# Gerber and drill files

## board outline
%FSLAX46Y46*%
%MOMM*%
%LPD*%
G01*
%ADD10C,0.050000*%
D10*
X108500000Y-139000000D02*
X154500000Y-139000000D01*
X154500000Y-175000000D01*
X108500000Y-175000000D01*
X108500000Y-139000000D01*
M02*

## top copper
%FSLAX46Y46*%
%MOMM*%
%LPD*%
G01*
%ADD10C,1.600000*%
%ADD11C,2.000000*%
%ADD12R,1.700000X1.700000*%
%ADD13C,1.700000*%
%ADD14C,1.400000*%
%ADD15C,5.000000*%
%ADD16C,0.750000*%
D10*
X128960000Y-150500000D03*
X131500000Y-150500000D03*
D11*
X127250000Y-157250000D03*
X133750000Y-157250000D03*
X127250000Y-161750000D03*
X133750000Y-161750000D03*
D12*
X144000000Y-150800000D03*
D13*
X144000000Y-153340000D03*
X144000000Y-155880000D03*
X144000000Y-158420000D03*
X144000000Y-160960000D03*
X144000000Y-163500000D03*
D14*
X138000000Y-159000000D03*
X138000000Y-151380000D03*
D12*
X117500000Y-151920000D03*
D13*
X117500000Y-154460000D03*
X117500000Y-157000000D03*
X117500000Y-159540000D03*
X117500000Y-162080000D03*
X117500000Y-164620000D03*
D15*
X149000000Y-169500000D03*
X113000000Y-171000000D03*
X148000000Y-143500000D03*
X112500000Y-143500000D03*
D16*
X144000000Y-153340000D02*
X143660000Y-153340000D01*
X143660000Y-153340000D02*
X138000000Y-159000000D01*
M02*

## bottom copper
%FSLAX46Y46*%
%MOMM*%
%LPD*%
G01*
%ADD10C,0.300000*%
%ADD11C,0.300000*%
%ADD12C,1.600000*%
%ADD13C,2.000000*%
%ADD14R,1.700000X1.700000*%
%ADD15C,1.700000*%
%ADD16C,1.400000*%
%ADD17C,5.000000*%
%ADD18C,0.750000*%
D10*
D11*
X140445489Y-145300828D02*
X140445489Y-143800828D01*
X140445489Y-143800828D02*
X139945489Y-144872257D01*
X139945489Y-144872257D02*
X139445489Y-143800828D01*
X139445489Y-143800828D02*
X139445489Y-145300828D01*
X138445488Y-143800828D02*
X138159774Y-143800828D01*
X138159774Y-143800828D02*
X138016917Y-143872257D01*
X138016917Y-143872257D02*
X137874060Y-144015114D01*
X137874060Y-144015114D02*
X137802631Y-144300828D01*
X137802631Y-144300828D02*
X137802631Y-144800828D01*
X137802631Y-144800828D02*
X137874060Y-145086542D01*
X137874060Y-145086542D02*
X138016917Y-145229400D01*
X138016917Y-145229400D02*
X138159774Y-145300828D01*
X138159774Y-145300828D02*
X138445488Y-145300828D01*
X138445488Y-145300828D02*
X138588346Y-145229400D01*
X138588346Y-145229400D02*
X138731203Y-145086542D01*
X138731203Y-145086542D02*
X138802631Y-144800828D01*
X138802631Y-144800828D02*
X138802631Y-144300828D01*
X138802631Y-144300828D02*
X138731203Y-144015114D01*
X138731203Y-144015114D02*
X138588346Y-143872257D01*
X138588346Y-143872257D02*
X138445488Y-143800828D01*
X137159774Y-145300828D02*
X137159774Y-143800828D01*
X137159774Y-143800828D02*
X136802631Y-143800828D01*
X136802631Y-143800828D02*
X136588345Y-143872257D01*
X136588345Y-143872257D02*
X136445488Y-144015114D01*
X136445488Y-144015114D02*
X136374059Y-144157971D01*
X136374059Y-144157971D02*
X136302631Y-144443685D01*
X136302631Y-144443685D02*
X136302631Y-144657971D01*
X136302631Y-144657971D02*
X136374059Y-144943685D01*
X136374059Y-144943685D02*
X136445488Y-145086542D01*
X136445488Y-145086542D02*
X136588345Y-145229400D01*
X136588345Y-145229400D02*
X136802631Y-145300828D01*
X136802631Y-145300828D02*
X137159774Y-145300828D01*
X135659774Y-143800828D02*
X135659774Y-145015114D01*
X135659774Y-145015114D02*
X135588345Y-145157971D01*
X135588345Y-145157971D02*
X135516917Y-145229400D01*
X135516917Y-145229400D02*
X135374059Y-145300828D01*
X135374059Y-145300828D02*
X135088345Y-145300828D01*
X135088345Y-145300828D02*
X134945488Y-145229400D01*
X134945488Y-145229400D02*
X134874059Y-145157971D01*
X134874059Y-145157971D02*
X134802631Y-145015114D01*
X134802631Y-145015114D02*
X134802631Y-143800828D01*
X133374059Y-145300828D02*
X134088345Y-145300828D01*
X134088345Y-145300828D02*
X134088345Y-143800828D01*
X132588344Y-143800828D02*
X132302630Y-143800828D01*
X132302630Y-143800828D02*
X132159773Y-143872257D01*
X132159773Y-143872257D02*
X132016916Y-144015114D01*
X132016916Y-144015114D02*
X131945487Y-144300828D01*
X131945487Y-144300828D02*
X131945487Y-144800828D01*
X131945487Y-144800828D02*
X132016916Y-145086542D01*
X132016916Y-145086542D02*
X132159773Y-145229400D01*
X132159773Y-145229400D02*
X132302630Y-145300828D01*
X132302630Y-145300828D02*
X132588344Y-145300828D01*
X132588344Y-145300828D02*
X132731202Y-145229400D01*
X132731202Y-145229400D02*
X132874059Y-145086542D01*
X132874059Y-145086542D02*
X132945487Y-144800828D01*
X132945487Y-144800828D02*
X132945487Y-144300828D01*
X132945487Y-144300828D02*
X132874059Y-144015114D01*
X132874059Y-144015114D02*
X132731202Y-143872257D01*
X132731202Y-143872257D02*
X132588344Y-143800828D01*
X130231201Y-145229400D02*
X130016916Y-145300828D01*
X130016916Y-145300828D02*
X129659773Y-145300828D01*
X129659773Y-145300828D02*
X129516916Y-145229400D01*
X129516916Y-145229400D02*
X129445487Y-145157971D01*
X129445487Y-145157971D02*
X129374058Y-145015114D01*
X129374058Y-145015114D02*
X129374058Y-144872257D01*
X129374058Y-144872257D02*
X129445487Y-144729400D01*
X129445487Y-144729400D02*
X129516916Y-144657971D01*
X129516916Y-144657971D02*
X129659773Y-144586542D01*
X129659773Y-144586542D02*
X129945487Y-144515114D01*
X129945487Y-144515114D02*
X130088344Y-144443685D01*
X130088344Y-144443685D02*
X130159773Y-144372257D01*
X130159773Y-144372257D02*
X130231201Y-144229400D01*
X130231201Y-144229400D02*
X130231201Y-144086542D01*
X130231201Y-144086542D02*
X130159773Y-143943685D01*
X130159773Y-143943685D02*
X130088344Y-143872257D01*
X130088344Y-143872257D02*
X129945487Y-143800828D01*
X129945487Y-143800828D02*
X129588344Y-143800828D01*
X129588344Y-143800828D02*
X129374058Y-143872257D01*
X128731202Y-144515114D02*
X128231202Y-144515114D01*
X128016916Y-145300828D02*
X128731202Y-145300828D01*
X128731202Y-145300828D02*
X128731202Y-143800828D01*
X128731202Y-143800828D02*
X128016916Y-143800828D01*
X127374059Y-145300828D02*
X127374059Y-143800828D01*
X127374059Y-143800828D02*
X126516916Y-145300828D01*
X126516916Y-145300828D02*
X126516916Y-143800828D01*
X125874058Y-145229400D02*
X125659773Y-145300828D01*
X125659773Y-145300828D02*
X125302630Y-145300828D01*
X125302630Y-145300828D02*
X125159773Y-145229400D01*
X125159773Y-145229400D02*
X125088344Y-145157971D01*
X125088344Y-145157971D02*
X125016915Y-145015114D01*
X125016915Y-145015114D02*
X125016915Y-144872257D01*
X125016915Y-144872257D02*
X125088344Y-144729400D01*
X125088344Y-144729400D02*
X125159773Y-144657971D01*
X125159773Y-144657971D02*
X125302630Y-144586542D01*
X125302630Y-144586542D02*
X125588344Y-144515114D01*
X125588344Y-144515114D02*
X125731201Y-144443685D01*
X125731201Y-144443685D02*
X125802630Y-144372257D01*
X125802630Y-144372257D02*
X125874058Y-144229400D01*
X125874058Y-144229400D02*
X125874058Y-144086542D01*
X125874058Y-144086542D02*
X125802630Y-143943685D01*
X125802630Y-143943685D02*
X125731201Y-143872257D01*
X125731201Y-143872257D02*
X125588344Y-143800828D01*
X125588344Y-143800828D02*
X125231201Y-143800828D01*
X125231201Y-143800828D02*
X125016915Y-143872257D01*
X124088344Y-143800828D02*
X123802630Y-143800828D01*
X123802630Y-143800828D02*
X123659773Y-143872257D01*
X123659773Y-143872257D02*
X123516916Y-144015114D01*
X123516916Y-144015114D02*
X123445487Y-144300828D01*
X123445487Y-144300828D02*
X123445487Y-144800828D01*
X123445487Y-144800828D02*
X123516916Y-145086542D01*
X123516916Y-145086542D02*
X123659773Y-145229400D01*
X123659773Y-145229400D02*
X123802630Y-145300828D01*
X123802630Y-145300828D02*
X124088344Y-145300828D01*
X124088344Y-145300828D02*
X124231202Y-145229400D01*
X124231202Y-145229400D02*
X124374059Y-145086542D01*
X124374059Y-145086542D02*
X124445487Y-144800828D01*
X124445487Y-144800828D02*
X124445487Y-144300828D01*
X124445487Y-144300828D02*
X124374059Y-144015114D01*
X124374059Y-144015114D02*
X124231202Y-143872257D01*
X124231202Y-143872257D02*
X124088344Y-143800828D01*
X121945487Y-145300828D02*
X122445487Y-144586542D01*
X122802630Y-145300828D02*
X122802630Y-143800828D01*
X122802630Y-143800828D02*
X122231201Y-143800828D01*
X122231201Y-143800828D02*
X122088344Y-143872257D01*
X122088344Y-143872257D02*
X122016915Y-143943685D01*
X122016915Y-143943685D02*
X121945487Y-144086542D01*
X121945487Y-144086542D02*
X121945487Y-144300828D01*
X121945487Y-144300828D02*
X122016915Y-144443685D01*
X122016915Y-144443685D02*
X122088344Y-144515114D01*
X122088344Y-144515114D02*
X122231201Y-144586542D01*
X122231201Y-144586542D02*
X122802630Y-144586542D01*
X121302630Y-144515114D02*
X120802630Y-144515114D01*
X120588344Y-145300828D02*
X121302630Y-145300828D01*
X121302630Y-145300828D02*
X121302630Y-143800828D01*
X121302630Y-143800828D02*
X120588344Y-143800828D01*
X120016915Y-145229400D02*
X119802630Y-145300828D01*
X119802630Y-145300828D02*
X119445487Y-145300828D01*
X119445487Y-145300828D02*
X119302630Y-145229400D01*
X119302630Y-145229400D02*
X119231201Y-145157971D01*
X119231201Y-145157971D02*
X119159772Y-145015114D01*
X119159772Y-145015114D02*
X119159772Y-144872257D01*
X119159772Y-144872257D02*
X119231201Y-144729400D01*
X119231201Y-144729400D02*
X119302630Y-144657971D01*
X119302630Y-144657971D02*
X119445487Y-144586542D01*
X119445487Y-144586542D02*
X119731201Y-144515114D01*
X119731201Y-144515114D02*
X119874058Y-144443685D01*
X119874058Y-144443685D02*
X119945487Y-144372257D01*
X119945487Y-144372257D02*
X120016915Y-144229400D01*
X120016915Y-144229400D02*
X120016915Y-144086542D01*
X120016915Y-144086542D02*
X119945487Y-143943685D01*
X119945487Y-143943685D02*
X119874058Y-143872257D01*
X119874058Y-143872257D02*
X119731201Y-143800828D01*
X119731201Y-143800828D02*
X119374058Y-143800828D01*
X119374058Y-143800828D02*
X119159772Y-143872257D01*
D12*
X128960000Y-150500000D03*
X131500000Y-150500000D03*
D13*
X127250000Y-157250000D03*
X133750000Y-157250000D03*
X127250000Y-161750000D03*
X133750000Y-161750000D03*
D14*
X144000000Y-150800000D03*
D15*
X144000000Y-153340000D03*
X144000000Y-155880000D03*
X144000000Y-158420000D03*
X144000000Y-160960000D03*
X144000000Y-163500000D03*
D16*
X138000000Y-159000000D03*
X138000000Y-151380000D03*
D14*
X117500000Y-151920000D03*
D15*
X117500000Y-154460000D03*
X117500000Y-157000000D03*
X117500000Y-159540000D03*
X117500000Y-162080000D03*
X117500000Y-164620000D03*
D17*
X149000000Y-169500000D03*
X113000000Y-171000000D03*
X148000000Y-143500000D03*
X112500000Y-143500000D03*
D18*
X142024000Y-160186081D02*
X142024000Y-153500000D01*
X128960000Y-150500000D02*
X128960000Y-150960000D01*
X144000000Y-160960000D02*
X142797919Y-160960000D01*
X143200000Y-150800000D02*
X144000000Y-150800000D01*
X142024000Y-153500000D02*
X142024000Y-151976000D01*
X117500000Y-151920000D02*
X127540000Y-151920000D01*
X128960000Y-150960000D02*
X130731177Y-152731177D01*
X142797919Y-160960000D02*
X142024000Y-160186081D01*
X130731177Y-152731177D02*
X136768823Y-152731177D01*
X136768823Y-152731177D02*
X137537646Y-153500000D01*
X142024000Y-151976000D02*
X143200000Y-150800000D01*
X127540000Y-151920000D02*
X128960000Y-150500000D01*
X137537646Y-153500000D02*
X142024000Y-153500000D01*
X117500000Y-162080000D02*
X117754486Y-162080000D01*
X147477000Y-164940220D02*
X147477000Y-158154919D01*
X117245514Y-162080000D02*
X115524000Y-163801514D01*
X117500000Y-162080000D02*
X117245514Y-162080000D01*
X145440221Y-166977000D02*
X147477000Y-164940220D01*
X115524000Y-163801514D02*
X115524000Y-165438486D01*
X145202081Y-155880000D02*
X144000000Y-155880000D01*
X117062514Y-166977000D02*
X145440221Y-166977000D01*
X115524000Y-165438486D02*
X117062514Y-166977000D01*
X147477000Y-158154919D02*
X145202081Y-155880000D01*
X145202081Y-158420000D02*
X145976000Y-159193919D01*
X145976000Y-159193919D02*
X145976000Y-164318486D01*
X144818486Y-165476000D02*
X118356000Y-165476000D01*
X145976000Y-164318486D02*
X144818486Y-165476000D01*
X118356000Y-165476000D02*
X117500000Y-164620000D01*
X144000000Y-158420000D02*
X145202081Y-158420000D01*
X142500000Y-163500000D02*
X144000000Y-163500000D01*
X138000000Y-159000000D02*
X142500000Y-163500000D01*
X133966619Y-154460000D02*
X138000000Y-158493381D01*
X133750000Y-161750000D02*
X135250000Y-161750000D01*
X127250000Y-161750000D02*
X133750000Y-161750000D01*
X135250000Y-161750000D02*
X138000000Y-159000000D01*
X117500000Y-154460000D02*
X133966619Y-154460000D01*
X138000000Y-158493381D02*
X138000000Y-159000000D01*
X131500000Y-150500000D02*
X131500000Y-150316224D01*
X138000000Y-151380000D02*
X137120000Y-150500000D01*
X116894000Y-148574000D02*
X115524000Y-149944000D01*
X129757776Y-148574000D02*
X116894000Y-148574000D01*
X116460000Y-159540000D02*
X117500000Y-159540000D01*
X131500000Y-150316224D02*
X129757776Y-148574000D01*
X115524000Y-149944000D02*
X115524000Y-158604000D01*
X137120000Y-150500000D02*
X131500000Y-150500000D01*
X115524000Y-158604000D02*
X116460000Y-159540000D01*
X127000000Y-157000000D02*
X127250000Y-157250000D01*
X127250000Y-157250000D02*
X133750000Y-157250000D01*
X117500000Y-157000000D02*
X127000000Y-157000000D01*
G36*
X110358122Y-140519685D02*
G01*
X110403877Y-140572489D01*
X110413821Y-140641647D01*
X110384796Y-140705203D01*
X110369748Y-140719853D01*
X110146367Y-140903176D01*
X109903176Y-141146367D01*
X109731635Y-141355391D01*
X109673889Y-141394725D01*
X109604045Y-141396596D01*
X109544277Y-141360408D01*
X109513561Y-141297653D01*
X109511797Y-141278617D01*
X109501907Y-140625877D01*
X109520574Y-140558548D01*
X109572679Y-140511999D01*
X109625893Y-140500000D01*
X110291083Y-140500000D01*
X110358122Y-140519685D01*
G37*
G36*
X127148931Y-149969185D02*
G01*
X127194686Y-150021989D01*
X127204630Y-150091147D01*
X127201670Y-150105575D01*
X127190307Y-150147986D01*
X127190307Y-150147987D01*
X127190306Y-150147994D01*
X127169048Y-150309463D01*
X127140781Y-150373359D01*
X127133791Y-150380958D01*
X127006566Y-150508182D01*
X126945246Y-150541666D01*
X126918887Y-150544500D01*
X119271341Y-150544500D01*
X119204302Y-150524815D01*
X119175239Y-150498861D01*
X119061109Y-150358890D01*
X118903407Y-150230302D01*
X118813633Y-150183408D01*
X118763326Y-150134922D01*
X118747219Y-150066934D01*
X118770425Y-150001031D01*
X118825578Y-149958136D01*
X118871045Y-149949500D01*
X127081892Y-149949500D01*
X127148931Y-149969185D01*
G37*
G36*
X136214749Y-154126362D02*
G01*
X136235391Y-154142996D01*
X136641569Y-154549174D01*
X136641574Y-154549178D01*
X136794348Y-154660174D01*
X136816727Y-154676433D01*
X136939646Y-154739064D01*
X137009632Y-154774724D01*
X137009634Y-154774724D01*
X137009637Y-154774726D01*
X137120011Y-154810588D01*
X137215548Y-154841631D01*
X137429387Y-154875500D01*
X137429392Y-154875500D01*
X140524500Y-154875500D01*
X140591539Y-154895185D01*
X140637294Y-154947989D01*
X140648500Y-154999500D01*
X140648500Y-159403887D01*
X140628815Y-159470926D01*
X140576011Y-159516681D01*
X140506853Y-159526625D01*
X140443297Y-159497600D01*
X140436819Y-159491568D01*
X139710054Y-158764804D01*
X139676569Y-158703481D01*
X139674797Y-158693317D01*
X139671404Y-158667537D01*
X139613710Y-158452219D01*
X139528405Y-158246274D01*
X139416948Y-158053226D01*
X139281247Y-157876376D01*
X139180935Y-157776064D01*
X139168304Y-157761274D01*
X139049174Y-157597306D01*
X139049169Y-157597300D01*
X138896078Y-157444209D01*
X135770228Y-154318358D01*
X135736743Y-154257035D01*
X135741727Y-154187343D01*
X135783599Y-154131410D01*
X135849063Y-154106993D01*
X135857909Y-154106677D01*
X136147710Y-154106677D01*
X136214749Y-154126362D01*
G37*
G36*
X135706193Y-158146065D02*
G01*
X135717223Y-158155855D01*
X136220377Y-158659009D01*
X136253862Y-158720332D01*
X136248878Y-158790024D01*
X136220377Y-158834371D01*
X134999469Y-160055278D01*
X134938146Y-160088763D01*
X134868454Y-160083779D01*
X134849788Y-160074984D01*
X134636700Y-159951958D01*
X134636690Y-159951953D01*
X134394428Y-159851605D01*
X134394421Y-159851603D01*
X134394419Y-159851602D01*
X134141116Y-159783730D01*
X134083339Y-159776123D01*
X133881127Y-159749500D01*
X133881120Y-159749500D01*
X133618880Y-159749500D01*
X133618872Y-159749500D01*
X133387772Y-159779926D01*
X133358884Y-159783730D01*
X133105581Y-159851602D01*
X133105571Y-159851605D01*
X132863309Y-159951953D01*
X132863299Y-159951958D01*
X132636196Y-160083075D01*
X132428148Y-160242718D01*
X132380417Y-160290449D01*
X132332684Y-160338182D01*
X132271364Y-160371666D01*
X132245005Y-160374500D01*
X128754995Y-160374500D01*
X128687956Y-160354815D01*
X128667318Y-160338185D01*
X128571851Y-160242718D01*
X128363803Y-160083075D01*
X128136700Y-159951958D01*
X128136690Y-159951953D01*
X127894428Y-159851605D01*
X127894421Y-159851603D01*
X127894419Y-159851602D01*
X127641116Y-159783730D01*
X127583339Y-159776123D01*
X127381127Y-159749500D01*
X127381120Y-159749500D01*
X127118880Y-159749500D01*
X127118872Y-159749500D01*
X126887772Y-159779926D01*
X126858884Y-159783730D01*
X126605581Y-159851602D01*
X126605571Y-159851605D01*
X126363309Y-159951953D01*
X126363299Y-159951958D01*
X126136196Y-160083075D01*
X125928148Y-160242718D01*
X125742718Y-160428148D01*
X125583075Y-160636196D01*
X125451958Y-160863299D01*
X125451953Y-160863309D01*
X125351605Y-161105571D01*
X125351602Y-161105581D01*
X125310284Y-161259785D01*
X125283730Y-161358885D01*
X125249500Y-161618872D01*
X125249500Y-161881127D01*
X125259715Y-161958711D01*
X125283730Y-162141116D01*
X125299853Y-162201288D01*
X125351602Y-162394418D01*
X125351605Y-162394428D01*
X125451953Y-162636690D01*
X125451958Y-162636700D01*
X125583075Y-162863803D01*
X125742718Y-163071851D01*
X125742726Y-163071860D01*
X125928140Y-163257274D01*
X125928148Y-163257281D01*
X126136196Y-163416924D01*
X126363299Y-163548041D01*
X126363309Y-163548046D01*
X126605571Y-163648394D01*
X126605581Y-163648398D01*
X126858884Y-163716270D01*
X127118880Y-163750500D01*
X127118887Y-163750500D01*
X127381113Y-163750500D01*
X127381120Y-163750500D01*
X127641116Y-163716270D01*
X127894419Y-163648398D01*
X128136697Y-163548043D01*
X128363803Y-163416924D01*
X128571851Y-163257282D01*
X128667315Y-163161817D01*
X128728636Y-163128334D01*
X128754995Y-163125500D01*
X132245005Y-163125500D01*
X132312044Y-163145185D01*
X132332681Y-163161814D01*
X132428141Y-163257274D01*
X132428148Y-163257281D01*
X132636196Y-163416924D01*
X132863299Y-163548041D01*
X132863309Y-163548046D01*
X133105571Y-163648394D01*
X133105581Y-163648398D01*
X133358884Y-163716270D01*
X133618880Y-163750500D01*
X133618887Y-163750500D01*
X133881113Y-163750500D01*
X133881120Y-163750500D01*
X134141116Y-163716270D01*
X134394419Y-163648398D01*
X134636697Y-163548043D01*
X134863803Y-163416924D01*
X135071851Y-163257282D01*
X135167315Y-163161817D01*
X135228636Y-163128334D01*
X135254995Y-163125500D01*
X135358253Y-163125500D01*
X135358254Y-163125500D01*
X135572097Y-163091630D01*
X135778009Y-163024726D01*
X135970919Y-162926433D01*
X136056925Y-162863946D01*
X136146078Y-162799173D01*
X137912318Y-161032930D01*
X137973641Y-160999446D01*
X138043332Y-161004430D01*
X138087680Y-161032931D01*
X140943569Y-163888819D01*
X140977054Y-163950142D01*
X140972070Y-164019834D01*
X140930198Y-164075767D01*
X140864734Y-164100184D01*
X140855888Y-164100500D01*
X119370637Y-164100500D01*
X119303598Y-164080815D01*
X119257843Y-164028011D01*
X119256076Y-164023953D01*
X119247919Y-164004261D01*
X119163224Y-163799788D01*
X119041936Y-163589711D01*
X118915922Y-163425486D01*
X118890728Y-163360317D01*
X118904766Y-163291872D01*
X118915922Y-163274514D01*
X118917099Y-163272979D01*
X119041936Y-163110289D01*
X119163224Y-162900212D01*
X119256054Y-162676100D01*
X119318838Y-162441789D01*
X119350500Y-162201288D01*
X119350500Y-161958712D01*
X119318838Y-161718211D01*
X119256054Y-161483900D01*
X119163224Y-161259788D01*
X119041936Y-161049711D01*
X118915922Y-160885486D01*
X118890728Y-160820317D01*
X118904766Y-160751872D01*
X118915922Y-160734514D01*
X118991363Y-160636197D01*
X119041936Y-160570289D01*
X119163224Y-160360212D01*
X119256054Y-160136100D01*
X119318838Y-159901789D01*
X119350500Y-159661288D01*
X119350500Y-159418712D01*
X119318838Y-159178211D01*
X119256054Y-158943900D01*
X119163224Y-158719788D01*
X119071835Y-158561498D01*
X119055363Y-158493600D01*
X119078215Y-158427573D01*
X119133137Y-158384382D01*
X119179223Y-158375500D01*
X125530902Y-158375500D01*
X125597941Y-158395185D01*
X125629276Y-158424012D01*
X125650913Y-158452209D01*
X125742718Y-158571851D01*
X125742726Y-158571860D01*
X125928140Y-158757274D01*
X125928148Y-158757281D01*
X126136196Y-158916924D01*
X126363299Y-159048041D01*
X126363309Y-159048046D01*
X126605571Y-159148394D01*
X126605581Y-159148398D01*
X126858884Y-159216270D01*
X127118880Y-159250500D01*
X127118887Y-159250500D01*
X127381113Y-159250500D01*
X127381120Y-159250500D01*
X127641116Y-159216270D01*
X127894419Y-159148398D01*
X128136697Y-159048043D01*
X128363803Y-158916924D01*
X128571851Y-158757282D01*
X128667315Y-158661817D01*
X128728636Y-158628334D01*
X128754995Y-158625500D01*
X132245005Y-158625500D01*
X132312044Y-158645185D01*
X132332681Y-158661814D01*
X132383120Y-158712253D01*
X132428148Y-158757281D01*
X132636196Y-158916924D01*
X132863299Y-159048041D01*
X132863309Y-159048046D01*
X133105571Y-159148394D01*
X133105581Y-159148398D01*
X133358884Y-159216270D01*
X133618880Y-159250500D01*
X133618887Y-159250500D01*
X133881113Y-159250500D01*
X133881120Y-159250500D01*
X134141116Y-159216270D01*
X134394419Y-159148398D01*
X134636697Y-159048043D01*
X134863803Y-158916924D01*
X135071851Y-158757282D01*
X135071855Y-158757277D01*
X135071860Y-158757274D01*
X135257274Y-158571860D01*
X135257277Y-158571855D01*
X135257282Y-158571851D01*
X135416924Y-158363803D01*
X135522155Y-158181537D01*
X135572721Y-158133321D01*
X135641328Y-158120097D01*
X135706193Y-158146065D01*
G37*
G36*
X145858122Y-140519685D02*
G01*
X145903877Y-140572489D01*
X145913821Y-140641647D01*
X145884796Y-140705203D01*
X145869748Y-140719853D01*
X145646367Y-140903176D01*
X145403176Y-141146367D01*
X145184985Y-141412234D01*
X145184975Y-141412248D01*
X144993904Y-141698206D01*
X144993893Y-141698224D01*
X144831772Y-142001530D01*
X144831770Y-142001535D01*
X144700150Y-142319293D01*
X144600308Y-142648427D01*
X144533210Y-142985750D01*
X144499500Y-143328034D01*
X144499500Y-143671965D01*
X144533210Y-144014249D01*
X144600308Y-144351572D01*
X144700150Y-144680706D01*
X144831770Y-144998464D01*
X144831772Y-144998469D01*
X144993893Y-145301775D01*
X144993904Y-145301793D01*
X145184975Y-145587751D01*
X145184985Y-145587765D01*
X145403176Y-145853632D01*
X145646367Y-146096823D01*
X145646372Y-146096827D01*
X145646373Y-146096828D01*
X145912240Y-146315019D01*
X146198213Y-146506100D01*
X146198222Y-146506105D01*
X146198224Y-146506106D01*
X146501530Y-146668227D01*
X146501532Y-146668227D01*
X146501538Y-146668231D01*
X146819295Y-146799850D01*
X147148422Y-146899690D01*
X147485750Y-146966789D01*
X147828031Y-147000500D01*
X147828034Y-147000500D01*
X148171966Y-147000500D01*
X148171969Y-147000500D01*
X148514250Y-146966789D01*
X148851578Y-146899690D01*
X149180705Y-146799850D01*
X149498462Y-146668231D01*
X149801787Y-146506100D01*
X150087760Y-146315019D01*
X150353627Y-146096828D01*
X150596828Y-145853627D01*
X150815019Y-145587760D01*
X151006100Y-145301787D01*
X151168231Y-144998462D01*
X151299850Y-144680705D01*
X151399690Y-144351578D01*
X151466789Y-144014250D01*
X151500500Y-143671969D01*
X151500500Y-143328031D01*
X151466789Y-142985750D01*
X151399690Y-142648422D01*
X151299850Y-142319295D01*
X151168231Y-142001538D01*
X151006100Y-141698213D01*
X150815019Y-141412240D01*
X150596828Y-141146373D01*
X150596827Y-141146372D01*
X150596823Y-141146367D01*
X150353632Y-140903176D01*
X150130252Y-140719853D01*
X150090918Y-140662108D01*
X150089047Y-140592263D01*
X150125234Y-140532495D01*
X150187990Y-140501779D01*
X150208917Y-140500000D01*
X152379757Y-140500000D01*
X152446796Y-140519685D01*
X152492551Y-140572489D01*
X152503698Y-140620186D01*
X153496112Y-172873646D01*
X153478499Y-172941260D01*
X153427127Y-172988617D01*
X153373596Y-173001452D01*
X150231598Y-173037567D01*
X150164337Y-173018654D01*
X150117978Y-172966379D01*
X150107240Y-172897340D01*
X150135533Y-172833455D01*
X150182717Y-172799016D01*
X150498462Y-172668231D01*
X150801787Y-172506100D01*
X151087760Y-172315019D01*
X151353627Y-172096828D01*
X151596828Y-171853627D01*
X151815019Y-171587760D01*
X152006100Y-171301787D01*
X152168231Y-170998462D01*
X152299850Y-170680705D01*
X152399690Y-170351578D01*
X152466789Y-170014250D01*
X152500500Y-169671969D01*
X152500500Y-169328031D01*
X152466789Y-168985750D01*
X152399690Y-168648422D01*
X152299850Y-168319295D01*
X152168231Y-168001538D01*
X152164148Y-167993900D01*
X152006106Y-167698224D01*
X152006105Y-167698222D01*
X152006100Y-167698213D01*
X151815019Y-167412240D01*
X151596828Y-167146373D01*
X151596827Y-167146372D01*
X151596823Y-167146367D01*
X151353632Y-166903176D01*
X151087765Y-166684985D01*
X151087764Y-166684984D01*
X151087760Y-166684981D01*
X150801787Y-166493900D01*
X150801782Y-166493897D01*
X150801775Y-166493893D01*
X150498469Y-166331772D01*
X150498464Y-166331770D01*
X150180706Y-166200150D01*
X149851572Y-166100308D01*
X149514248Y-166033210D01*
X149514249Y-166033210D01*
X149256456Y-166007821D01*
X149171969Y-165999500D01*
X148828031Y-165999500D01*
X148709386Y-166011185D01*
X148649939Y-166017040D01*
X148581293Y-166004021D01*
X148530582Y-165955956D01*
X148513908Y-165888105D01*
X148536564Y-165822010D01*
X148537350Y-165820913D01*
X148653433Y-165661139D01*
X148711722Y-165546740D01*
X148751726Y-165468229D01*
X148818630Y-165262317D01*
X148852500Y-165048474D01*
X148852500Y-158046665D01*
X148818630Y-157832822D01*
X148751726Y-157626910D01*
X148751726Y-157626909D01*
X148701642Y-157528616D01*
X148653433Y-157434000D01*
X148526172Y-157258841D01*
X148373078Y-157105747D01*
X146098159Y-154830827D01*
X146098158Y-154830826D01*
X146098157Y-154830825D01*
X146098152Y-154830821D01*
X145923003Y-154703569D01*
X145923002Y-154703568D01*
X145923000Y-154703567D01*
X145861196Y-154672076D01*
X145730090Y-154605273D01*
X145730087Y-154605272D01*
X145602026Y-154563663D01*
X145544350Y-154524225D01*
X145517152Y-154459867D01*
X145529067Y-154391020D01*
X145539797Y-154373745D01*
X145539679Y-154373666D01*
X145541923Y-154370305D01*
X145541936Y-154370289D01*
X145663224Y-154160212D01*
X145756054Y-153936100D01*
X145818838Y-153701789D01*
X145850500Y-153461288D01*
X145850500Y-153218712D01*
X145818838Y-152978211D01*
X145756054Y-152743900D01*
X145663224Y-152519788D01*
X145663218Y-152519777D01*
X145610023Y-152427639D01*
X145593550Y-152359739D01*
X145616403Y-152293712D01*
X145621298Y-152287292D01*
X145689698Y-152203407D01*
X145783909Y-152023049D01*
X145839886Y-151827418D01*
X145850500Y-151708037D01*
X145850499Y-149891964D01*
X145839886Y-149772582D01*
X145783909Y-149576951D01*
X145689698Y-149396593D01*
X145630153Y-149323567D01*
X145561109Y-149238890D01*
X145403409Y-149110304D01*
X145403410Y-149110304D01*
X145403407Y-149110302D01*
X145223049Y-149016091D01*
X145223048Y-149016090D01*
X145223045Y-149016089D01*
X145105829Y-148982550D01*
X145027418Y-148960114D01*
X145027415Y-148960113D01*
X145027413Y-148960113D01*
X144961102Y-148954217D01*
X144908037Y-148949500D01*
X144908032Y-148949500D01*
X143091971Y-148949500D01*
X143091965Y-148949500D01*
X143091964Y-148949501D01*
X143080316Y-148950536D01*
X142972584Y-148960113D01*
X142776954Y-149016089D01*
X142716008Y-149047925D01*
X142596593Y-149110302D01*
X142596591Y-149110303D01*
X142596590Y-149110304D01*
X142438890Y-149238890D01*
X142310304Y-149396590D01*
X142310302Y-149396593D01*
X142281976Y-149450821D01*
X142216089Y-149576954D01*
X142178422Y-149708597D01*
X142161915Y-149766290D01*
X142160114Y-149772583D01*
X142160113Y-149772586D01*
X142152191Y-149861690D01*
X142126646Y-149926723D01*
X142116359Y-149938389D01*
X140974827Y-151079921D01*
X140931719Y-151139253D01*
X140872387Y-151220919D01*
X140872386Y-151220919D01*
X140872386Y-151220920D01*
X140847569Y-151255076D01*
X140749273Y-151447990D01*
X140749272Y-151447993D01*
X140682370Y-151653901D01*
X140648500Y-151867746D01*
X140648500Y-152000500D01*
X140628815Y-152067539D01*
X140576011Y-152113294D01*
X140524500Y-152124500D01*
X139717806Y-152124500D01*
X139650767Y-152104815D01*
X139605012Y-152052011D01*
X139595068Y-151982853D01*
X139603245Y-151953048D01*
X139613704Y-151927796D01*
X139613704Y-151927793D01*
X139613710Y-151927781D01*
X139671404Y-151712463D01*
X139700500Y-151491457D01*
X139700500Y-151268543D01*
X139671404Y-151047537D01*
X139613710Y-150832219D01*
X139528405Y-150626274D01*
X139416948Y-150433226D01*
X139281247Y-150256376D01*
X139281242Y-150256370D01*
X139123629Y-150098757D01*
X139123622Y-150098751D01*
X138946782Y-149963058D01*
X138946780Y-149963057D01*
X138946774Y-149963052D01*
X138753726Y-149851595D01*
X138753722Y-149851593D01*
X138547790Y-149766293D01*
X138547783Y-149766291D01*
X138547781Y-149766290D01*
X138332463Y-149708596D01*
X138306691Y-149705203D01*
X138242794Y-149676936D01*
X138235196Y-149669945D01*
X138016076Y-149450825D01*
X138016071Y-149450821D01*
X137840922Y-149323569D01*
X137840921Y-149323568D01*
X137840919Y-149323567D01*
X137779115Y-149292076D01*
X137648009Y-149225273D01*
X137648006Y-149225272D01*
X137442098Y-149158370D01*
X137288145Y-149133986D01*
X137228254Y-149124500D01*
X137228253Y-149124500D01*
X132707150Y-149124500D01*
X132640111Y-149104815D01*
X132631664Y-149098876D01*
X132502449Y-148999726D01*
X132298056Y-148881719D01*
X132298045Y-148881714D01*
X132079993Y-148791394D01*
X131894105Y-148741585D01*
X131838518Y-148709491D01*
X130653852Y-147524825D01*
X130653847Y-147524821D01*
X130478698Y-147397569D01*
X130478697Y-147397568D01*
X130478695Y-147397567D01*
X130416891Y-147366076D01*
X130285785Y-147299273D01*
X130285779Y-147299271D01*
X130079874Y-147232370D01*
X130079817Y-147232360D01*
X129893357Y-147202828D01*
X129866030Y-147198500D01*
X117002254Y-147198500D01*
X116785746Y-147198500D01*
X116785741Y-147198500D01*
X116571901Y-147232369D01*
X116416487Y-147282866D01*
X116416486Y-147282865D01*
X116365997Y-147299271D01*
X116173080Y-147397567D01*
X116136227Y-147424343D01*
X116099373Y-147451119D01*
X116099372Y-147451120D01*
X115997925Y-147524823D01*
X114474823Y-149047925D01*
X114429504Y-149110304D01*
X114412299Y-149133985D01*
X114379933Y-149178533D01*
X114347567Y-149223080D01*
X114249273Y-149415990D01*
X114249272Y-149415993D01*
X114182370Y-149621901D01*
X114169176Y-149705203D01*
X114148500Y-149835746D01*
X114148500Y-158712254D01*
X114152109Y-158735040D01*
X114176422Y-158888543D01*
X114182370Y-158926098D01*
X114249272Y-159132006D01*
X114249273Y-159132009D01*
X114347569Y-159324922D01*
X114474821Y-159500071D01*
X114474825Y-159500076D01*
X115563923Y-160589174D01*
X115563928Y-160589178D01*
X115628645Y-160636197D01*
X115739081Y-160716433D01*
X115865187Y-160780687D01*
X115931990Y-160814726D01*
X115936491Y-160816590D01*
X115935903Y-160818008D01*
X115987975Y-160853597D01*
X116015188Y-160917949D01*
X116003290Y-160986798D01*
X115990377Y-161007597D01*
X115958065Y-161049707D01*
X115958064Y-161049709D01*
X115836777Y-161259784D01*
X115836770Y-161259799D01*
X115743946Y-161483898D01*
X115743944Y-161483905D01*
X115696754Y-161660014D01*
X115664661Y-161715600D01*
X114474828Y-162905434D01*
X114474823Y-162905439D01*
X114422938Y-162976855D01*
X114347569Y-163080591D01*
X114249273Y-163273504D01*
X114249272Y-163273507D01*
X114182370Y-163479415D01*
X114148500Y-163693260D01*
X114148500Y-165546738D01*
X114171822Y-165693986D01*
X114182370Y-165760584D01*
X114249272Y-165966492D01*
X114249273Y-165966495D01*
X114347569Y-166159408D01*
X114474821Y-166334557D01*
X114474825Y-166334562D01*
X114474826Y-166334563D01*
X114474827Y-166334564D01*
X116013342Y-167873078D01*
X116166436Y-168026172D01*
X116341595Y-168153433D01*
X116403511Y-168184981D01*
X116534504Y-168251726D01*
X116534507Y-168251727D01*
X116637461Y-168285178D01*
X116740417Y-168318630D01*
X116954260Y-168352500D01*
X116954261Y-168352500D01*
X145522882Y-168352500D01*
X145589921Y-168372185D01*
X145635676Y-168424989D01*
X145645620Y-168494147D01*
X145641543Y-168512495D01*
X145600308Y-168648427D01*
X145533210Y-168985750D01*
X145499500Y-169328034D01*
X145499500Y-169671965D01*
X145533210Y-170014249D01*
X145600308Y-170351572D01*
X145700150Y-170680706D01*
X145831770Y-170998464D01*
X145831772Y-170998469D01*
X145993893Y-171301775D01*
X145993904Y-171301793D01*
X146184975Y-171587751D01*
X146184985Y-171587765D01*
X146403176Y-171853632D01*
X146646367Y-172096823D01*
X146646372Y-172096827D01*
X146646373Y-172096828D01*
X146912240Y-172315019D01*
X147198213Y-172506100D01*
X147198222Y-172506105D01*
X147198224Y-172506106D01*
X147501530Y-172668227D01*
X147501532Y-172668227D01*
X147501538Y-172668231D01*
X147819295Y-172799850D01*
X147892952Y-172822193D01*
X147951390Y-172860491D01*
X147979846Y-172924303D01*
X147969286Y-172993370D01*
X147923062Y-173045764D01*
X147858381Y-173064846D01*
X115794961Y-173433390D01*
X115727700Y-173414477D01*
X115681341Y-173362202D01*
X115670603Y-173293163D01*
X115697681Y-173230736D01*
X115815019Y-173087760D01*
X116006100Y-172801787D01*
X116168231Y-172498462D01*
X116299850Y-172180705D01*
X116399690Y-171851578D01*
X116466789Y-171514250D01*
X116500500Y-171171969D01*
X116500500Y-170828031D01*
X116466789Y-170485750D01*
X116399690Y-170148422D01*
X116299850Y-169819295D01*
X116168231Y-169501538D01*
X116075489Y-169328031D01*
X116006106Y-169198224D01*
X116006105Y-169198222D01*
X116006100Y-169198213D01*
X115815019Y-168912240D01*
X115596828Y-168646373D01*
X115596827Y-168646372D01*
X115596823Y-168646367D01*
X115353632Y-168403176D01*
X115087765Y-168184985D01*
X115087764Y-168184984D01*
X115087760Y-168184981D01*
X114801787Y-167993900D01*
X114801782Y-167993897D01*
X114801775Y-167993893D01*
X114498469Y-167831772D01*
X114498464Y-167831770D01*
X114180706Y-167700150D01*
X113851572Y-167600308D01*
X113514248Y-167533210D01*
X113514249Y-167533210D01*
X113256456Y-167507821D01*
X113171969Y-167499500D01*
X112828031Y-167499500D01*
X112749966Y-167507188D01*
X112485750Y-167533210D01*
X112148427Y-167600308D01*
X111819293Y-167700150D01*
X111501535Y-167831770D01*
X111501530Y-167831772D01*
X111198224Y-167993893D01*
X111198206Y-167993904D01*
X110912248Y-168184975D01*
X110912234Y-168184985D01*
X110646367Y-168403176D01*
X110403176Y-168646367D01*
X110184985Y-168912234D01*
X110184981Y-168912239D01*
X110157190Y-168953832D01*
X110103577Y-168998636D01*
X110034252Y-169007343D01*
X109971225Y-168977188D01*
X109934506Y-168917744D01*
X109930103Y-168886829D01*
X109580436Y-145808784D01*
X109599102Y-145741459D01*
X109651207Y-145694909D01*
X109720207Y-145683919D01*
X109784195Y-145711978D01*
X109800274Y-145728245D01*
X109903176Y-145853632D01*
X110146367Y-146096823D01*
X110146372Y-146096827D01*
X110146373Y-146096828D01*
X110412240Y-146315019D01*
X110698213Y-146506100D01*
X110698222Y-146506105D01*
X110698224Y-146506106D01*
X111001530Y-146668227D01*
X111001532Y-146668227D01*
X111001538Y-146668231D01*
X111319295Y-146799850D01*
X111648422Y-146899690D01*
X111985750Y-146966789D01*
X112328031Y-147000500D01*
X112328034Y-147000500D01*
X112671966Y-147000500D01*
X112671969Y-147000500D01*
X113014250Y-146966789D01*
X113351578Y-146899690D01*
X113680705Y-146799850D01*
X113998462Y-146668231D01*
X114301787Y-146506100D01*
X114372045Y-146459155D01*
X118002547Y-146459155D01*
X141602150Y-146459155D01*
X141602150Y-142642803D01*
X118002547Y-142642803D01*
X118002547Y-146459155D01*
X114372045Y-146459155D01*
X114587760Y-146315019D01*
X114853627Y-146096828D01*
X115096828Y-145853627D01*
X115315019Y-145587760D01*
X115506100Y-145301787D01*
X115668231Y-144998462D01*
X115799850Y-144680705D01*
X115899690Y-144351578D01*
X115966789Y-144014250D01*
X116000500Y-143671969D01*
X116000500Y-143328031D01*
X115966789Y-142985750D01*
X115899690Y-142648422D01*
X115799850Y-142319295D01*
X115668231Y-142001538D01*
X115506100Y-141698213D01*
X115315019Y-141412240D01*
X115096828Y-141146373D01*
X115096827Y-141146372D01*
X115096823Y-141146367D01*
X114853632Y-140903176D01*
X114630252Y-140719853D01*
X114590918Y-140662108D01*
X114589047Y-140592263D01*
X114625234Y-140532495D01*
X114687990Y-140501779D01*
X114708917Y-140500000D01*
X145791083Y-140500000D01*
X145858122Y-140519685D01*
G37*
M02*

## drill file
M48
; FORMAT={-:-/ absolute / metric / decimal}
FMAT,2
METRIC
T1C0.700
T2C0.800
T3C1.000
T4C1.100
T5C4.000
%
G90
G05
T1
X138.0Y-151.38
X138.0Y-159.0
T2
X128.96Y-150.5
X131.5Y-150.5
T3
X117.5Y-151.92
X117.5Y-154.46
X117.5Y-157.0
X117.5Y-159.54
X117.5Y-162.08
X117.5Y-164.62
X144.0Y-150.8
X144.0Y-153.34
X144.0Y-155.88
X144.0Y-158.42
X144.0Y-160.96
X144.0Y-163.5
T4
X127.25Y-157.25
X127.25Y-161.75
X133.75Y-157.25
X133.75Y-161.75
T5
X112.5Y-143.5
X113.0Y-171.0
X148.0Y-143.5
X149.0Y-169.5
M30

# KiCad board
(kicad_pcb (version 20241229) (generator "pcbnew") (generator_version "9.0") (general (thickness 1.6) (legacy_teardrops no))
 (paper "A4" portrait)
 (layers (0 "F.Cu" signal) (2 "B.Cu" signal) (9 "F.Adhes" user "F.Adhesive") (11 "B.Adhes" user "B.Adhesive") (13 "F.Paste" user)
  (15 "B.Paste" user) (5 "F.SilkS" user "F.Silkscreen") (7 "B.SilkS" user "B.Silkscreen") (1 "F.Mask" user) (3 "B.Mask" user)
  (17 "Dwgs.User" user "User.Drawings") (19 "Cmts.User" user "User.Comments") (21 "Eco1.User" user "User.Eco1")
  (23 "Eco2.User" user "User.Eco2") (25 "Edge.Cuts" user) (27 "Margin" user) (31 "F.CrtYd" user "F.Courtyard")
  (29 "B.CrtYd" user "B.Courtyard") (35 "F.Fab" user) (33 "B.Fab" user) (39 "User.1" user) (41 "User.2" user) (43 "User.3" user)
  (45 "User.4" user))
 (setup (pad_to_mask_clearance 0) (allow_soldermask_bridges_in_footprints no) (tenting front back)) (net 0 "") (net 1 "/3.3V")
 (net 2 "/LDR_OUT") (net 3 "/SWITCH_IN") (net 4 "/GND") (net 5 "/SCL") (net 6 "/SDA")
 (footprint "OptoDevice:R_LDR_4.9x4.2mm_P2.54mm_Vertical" (layer "F.Cu") (at 128.96 150.5)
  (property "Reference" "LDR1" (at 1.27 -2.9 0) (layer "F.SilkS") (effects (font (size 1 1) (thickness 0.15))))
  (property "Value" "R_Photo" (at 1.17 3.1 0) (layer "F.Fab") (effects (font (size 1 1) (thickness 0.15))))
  (pad "1" thru_hole circle (at 0 0) (size 1.6 1.6) (drill 0.8) (layers "*.Cu" "*.Mask") (remove_unused_layers no) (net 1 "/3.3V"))
  (pad "2" thru_hole circle (at 2.54 0) (size 1.6 1.6) (drill 0.8) (layers "*.Cu" "*.Mask") (remove_unused_layers no) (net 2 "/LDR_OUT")))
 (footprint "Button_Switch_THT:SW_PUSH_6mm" (layer "F.Cu") (at 127.25 157.25)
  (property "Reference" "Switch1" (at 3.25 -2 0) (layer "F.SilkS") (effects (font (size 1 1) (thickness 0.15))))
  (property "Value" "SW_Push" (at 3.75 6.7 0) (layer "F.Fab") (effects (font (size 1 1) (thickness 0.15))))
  (pad "1" thru_hole circle (at 0 0 90) (size 2 2) (drill 1.1) (layers "*.Cu" "*.Mask") (remove_unused_layers no) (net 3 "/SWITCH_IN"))
  (pad "1" thru_hole circle (at 6.5 0 90) (size 2 2) (drill 1.1) (layers "*.Cu" "*.Mask") (remove_unused_layers no) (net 3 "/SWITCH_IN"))
  (pad "2" thru_hole circle (at 0 4.5 90) (size 2 2) (drill 1.1) (layers "*.Cu" "*.Mask") (remove_unused_layers no) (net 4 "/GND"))
  (pad "2" thru_hole circle (at 6.5 4.5 90) (size 2 2) (drill 1.1) (layers "*.Cu" "*.Mask") (remove_unused_layers no) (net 4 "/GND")))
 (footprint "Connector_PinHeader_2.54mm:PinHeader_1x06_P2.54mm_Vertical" (layer "F.Cu") (at 144 150.8)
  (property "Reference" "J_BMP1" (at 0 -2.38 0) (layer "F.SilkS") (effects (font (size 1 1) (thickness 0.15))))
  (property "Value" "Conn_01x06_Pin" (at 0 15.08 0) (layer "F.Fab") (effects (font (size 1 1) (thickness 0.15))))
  (pad "1" thru_hole rect (at 0 0) (size 1.7 1.7) (drill 1) (layers "*.Cu" "*.Mask") (remove_unused_layers no) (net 1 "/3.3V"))
  (pad "2" thru_hole circle (at 0 2.54) (size 1.7 1.7) (drill 1) (layers "*.Cu" "*.Mask") (remove_unused_layers no) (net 4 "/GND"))
  (pad "3" thru_hole circle (at 0 5.08) (size 1.7 1.7) (drill 1) (layers "*.Cu" "*.Mask") (remove_unused_layers no) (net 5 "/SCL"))
  (pad "4" thru_hole circle (at 0 7.62) (size 1.7 1.7) (drill 1) (layers "*.Cu" "*.Mask") (remove_unused_layers no) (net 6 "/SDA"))
  (pad "5" thru_hole circle (at 0 10.16) (size 1.7 1.7) (drill 1) (layers "*.Cu" "*.Mask") (remove_unused_layers no) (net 1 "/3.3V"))
  (pad "6" thru_hole circle (at 0 12.7) (size 1.7 1.7) (drill 1) (layers "*.Cu" "*.Mask") (remove_unused_layers no) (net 4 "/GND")))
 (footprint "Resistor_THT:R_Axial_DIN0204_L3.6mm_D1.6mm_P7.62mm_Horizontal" (layer "F.Cu") (at 138 159 90)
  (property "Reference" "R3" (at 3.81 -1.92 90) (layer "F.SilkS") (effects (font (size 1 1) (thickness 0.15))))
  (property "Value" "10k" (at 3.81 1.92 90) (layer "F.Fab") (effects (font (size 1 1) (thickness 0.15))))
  (pad "1" thru_hole circle (at 0 0 90) (size 1.4 1.4) (drill 0.7) (layers "*.Cu" "*.Mask") (remove_unused_layers no) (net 4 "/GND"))
  (pad "2" thru_hole circle (at 7.62 0 90) (size 1.4 1.4) (drill 0.7) (layers "*.Cu" "*.Mask") (remove_unused_layers no) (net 2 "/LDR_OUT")))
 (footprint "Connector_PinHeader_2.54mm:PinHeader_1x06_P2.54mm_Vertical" (layer "F.Cu") (at 117.5 151.92)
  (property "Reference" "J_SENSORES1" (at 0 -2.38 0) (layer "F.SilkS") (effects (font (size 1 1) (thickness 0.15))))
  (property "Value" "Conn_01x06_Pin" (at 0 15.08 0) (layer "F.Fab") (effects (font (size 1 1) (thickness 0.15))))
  (pad "1" thru_hole rect (at 0 0) (size 1.7 1.7) (drill 1) (layers "*.Cu" "*.Mask") (remove_unused_layers no) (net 1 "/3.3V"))
  (pad "2" thru_hole circle (at 0 2.54) (size 1.7 1.7) (drill 1) (layers "*.Cu" "*.Mask") (remove_unused_layers no) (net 4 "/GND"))
  (pad "3" thru_hole circle (at 0 5.08) (size 1.7 1.7) (drill 1) (layers "*.Cu" "*.Mask") (remove_unused_layers no) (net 3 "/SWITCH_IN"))
  (pad "4" thru_hole circle (at 0 7.62) (size 1.7 1.7) (drill 1) (layers "*.Cu" "*.Mask") (remove_unused_layers no) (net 2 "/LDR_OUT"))
  (pad "5" thru_hole circle (at 0 10.16) (size 1.7 1.7) (drill 1) (layers "*.Cu" "*.Mask") (remove_unused_layers no) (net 5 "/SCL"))
  (pad "6" thru_hole circle (at 0 12.7) (size 1.7 1.7) (drill 1) (layers "*.Cu" "*.Mask") (remove_unused_layers no) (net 6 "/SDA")))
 (gr_rect (start 108.5 139) (end 154.5 175) (stroke (width 0.05) (type default)) (fill no) (layer "Edge.Cuts"))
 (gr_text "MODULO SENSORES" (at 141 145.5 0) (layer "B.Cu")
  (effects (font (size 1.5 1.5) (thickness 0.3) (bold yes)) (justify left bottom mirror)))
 (via (at 149 169.5) (size 5) (drill 4) (layers "F.Cu" "B.Cu") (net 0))
 (via (at 113 171) (size 5) (drill 4) (layers "F.Cu" "B.Cu") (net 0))
 (via (at 148 143.5) (size 5) (drill 4) (layers "F.Cu" "B.Cu") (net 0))
 (via (at 112.5 143.5) (size 5) (drill 4) (layers "F.Cu" "B.Cu") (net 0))
 (segment (start 142.024 160.186081) (end 142.024 153.5) (width 0.75) (layer "B.Cu") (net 1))
 (segment (start 128.96 150.5) (end 128.96 150.96) (width 0.75) (layer "B.Cu") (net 1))
 (segment (start 144 160.96) (end 142.797919 160.96) (width 0.75) (layer "B.Cu") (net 1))
 (segment (start 143.2 150.8) (end 144 150.8) (width 0.75) (layer "B.Cu") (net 1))
 (segment (start 142.024 153.5) (end 142.024 151.976) (width 0.75) (layer "B.Cu") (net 1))
 (segment (start 117.5 151.92) (end 127.54 151.92) (width 0.75) (layer "B.Cu") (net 1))
 (segment (start 128.96 150.96) (end 130.731177 152.731177) (width 0.75) (layer "B.Cu") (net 1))
 (segment (start 142.797919 160.96) (end 142.024 160.186081) (width 0.75) (layer "B.Cu") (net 1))
 (segment (start 130.731177 152.731177) (end 136.768823 152.731177) (width 0.75) (layer "B.Cu") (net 1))
 (segment (start 136.768823 152.731177) (end 137.537646 153.5) (width 0.75) (layer "B.Cu") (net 1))
 (segment (start 142.024 151.976) (end 143.2 150.8) (width 0.75) (layer "B.Cu") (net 1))
 (segment (start 127.54 151.92) (end 128.96 150.5) (width 0.75) (layer "B.Cu") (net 1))
 (segment (start 137.537646 153.5) (end 142.024 153.5) (width 0.75) (layer "B.Cu") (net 1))
 (segment (start 117.5 162.08) (end 117.754486 162.08) (width 0.75) (layer "B.Cu") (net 5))
 (segment (start 147.477 164.94022) (end 147.477 158.154919) (width 0.75) (layer "B.Cu") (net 5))
 (segment (start 117.245514 162.08) (end 115.524 163.801514) (width 0.75) (layer "B.Cu") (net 5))
 (segment (start 117.5 162.08) (end 117.245514 162.08) (width 0.75) (layer "B.Cu") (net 5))
 (segment (start 145.440221 166.977) (end 147.477 164.94022) (width 0.75) (layer "B.Cu") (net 5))
 (segment (start 115.524 163.801514) (end 115.524 165.438486) (width 0.75) (layer "B.Cu") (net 5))
 (segment (start 145.202081 155.88) (end 144 155.88) (width 0.75) (layer "B.Cu") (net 5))
 (segment (start 117.062514 166.977) (end 145.440221 166.977) (width 0.75) (layer "B.Cu") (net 5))
 (segment (start 115.524 165.438486) (end 117.062514 166.977) (width 0.75) (layer "B.Cu") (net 5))
 (segment (start 147.477 158.154919) (end 145.202081 155.88) (width 0.75) (layer "B.Cu") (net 5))
 (segment (start 145.202081 158.42) (end 145.976 159.193919) (width 0.75) (layer "B.Cu") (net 6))
 (segment (start 145.976 159.193919) (end 145.976 164.318486) (width 0.75) (layer "B.Cu") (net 6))
 (segment (start 144.818486 165.476) (end 118.356 165.476) (width 0.75) (layer "B.Cu") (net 6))
 (segment (start 145.976 164.318486) (end 144.818486 165.476) (width 0.75) (layer "B.Cu") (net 6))
 (segment (start 118.356 165.476) (end 117.5 164.62) (width 0.75) (layer "B.Cu") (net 6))
 (segment (start 144 158.42) (end 145.202081 158.42) (width 0.75) (layer "B.Cu") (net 6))
 (segment (start 144 153.34) (end 143.66 153.34) (width 0.75) (layer "F.Cu") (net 4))
 (segment (start 143.66 153.34) (end 138 159) (width 0.75) (layer "F.Cu") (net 4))
 (segment (start 142.5 163.5) (end 144 163.5) (width 0.75) (layer "B.Cu") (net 4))
 (segment (start 138 159) (end 142.5 163.5) (width 0.75) (layer "B.Cu") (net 4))
 (segment (start 133.966619 154.46) (end 138 158.493381) (width 0.75) (layer "B.Cu") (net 4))
 (segment (start 133.75 161.75) (end 135.25 161.75) (width 0.75) (layer "B.Cu") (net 4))
 (segment (start 127.25 161.75) (end 133.75 161.75) (width 0.75) (layer "B.Cu") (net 4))
 (segment (start 135.25 161.75) (end 138 159) (width 0.75) (layer "B.Cu") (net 4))
 (segment (start 117.5 154.46) (end 133.966619 154.46) (width 0.75) (layer "B.Cu") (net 4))
 (segment (start 138 158.493381) (end 138 159) (width 0.75) (layer "B.Cu") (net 4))
 (segment (start 131.5 150.5) (end 131.5 150.316224) (width 0.75) (layer "B.Cu") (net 2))
 (segment (start 138 151.38) (end 137.12 150.5) (width 0.75) (layer "B.Cu") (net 2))
 (segment (start 116.894 148.574) (end 115.524 149.944) (width 0.75) (layer "B.Cu") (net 2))
 (segment (start 129.757776 148.574) (end 116.894 148.574) (width 0.75) (layer "B.Cu") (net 2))
 (segment (start 116.46 159.54) (end 117.5 159.54) (width 0.75) (layer "B.Cu") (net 2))
 (segment (start 131.5 150.316224) (end 129.757776 148.574) (width 0.75) (layer "B.Cu") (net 2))
 (segment (start 115.524 149.944) (end 115.524 158.604) (width 0.75) (layer "B.Cu") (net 2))
 (segment (start 137.12 150.5) (end 131.5 150.5) (width 0.75) (layer "B.Cu") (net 2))
 (segment (start 115.524 158.604) (end 116.46 159.54) (width 0.75) (layer "B.Cu") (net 2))
 (segment (start 127 157) (end 127.25 157.25) (width 0.75) (layer "B.Cu") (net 3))
 (segment (start 127.25 157.25) (end 133.75 157.25) (width 0.75) (layer "B.Cu") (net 3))
 (segment (start 117.5 157) (end 127 157) (width 0.75) (layer "B.Cu") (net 3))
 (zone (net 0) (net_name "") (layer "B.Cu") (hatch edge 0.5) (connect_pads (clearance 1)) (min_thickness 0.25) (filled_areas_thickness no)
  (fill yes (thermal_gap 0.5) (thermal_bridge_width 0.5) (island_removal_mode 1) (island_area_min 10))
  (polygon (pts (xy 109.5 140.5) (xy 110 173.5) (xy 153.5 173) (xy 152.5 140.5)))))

